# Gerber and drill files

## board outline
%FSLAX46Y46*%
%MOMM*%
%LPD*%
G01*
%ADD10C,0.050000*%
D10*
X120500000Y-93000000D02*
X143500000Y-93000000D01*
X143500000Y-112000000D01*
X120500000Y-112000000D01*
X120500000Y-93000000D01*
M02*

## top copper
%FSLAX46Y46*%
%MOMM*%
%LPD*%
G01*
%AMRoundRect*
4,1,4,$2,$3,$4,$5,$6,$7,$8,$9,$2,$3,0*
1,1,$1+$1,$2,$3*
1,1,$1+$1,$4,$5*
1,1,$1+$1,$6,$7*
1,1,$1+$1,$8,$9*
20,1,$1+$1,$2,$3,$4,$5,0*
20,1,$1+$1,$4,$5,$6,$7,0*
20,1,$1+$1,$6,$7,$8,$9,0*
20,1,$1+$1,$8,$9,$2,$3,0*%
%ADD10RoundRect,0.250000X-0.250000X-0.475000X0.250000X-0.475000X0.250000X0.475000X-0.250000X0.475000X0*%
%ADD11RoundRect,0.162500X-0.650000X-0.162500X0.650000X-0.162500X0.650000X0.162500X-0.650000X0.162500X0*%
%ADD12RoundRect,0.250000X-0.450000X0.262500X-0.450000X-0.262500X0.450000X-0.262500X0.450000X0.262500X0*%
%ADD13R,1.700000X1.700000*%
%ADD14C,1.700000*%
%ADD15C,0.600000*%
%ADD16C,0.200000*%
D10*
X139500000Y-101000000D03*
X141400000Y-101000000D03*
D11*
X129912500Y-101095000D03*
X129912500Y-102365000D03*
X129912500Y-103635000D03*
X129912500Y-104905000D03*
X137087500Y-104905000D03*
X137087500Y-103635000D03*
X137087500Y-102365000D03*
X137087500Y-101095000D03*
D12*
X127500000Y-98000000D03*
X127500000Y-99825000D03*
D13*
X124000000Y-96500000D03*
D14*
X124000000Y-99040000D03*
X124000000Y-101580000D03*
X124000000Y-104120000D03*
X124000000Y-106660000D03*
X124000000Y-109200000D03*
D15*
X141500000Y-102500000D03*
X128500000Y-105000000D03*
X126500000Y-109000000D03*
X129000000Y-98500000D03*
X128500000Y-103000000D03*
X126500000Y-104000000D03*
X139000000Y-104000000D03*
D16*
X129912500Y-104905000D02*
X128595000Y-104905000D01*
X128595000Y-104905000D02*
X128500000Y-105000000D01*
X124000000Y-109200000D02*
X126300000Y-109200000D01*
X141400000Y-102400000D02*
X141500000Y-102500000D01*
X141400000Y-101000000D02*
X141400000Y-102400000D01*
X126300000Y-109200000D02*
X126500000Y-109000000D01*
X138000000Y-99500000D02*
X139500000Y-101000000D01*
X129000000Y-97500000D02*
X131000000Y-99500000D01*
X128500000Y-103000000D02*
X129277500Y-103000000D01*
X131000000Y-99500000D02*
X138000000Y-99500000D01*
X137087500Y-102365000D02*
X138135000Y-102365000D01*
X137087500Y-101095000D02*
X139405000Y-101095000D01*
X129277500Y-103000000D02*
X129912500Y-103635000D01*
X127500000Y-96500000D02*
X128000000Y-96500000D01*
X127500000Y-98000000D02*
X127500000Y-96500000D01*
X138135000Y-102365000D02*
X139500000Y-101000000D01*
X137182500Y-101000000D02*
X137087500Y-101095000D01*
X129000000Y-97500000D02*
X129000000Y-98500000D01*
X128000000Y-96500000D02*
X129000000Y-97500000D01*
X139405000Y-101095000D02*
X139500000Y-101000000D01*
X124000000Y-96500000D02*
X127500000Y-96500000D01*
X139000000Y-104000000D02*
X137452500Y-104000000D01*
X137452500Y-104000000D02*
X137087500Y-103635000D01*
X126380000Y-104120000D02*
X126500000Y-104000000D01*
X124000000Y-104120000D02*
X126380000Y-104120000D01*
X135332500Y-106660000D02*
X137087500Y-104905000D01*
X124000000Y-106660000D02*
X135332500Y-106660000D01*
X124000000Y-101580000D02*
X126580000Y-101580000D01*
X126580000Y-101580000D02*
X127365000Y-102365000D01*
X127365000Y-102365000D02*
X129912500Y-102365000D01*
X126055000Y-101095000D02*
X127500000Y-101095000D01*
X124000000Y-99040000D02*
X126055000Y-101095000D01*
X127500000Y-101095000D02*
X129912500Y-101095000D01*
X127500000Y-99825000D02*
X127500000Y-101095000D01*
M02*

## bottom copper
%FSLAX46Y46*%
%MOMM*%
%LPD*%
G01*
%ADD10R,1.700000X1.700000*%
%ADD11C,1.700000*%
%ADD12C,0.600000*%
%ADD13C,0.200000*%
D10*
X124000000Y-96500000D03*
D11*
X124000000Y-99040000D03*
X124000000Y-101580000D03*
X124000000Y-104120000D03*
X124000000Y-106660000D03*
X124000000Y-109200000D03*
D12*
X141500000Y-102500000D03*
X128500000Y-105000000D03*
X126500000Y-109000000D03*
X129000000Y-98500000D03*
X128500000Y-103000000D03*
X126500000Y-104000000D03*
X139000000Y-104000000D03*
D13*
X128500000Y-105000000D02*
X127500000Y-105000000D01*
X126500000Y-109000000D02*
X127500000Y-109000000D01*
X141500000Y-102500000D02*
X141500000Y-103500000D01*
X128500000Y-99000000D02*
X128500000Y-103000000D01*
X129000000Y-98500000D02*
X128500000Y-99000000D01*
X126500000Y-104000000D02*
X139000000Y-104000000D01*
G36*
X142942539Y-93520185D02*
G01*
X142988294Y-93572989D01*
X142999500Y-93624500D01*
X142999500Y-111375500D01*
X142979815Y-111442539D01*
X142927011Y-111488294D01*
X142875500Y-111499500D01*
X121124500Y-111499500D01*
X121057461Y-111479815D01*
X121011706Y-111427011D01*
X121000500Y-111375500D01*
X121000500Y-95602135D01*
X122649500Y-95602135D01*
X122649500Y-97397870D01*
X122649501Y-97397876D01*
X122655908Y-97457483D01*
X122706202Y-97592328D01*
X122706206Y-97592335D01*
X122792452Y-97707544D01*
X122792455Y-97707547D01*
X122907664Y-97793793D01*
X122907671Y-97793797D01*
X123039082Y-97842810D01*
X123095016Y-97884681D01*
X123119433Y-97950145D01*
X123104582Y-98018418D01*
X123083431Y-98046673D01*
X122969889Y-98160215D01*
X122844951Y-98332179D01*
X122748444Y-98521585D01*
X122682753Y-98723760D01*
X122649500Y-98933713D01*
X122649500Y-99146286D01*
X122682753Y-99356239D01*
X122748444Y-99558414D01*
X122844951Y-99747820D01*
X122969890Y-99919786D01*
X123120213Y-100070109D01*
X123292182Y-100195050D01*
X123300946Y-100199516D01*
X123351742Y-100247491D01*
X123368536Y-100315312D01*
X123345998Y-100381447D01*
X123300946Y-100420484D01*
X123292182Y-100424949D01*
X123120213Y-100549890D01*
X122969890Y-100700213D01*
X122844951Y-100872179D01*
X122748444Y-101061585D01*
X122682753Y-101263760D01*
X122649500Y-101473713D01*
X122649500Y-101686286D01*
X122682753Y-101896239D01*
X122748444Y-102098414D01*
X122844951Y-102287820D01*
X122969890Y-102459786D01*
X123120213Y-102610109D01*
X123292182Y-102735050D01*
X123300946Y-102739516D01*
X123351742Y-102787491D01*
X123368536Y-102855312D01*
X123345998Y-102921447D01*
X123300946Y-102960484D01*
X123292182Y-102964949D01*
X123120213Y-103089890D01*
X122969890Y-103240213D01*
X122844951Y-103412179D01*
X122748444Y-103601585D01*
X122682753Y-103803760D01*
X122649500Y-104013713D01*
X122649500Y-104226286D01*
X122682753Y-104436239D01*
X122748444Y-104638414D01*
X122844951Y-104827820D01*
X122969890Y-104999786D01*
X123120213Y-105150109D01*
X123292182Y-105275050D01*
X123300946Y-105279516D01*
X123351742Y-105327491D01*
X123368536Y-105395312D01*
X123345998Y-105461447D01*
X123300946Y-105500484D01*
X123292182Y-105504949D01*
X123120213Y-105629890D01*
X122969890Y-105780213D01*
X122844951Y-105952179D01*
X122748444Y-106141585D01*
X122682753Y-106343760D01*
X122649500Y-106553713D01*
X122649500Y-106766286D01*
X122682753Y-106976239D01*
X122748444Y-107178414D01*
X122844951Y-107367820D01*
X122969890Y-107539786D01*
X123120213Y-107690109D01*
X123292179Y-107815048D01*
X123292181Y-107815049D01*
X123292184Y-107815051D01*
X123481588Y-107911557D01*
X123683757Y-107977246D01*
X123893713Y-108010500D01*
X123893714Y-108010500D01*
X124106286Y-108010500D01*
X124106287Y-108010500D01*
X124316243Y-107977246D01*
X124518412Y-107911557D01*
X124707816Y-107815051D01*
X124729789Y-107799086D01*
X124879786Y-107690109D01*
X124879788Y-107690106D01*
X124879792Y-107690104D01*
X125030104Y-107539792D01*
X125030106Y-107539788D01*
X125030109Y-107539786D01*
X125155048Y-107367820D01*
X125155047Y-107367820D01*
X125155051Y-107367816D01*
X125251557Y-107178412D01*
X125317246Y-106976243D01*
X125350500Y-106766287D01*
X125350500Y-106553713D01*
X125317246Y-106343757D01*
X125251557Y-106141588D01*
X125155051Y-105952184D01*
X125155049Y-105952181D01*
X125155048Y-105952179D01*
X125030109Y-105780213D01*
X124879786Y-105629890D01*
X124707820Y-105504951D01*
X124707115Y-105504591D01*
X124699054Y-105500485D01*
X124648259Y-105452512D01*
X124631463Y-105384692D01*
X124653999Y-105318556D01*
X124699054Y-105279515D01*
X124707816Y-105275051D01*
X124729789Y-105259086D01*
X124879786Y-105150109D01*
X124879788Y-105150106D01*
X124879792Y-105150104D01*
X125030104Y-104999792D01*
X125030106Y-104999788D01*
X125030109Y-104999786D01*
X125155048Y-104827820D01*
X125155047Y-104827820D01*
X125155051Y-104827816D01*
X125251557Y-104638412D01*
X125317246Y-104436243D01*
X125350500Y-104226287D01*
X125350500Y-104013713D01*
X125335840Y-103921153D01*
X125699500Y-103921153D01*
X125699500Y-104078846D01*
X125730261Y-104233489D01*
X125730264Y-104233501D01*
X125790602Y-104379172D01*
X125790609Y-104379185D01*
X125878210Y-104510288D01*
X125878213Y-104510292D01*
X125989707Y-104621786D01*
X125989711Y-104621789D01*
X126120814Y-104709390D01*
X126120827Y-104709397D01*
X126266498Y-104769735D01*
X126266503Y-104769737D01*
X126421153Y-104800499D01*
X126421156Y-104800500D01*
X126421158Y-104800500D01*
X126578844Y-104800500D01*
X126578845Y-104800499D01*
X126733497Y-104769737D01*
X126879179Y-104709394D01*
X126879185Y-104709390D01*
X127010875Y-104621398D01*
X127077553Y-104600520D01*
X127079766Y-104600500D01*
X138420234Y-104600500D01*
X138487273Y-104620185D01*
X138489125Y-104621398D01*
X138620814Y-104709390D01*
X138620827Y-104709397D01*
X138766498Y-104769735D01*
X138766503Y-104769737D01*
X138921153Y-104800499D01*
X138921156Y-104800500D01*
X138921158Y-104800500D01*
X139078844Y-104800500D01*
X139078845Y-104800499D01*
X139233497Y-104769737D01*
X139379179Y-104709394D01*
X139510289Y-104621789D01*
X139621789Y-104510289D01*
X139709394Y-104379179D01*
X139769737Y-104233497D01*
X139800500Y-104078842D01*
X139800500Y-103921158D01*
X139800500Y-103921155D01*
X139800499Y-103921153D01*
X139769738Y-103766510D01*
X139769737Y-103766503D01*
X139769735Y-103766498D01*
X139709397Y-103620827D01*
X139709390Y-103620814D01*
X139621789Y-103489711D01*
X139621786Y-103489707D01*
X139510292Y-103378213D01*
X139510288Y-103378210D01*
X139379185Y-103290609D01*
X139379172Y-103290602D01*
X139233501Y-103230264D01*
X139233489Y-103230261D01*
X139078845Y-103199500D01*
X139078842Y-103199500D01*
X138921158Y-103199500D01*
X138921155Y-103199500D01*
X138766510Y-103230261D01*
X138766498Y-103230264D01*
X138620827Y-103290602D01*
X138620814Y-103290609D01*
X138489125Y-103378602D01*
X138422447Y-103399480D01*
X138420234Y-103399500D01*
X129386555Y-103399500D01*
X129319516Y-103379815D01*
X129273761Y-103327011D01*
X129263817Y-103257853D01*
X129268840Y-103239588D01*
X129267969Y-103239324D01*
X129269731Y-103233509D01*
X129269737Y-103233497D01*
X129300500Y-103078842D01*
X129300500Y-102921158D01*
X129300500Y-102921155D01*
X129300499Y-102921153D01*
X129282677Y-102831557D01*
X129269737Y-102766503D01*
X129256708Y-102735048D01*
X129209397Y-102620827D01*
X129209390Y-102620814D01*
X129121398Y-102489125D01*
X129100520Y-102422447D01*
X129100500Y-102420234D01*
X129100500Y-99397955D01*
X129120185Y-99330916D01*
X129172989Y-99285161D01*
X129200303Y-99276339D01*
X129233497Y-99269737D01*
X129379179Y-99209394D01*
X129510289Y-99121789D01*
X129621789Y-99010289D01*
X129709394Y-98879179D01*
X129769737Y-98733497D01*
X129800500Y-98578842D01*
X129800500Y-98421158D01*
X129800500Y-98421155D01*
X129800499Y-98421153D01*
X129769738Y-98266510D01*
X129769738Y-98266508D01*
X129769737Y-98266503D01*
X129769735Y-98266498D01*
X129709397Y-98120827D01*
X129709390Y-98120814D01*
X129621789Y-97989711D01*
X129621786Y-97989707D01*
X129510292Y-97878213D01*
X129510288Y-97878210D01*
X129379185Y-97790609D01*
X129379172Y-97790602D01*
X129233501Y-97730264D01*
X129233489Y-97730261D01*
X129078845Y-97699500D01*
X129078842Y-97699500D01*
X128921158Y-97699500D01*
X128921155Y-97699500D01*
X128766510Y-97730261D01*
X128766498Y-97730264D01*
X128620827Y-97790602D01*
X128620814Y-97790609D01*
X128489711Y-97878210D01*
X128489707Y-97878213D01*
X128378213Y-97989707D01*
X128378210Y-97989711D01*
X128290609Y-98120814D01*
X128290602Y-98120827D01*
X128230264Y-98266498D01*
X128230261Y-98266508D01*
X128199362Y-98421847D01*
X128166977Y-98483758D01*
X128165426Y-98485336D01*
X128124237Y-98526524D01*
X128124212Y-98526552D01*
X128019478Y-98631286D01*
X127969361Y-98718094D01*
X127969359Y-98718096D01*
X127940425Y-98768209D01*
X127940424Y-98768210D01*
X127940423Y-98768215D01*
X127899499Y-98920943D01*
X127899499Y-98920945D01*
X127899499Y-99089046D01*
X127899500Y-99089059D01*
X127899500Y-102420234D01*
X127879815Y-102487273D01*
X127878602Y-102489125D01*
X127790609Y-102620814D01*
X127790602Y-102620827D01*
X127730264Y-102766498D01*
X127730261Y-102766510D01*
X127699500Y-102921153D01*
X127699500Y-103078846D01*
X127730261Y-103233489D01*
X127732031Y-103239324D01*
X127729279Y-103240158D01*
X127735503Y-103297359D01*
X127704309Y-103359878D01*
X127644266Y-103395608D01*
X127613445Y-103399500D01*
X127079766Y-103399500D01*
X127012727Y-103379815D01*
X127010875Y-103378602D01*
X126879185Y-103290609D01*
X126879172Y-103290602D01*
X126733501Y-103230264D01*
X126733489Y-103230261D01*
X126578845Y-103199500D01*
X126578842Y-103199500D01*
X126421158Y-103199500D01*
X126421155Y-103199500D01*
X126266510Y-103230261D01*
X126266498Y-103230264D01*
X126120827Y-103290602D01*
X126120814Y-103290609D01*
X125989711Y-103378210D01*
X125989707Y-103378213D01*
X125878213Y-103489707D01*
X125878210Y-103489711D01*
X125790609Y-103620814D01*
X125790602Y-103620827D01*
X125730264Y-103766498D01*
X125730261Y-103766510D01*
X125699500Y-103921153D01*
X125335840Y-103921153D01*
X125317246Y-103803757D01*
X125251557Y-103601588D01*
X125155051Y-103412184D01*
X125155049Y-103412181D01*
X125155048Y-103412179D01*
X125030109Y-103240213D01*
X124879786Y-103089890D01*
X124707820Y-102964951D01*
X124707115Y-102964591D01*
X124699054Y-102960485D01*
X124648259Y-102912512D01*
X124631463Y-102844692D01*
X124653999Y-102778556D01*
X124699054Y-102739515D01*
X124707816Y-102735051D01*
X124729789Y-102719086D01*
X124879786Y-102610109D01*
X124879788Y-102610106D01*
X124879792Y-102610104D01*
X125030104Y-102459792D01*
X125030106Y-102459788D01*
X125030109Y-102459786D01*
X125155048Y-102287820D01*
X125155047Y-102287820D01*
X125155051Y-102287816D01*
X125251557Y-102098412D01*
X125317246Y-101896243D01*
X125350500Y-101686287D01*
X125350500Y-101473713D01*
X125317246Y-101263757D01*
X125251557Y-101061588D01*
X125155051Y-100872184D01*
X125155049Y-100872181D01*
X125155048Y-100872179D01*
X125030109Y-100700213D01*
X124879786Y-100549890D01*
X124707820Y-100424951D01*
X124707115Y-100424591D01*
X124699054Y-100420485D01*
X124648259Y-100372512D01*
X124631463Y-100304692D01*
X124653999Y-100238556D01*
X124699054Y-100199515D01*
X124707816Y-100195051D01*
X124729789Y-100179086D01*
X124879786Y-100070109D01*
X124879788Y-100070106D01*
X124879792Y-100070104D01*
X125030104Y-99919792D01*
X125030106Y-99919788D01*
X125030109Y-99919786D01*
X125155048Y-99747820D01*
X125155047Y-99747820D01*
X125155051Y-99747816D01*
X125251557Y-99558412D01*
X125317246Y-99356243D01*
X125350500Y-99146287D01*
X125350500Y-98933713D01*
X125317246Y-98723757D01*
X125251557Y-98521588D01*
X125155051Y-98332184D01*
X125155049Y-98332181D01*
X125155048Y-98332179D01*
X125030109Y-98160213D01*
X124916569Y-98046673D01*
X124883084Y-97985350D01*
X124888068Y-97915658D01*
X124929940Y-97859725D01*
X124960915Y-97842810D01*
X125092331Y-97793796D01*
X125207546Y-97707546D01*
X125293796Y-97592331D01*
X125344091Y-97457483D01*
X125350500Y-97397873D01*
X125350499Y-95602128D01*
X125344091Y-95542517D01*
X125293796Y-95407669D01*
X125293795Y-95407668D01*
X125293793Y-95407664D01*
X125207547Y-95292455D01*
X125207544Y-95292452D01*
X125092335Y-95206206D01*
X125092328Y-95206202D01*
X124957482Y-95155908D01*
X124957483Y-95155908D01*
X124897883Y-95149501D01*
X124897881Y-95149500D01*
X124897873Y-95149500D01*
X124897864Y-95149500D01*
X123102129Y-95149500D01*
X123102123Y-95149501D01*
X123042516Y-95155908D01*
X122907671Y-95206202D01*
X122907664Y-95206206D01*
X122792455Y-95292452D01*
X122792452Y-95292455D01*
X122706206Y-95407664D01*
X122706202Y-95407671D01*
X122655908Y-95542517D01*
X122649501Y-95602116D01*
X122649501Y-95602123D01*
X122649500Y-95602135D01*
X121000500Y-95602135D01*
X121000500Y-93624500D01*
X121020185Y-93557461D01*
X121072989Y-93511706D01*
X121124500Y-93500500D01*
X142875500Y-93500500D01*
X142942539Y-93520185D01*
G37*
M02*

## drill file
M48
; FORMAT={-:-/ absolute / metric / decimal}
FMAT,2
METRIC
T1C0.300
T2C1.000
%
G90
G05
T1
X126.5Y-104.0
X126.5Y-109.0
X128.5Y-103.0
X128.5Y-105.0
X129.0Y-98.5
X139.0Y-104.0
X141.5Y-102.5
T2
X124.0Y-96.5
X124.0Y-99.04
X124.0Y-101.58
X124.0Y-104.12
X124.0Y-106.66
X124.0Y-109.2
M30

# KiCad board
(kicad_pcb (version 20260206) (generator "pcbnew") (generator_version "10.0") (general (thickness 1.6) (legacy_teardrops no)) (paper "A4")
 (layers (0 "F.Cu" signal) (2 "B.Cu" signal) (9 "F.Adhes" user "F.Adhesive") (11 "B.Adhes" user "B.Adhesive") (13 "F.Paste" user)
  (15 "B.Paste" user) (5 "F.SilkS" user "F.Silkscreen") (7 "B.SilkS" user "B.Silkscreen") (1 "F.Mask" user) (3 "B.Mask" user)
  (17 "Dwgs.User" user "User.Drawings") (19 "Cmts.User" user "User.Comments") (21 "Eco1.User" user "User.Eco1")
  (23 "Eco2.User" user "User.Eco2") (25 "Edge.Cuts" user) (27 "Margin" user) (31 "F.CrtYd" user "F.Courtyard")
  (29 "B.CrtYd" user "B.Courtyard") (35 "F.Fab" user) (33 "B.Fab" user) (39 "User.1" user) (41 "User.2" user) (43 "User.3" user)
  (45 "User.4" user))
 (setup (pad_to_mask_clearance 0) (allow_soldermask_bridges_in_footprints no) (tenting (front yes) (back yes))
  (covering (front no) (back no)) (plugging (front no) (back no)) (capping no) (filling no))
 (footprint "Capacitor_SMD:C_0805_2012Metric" (layer "F.Cu") (at 140.45 101)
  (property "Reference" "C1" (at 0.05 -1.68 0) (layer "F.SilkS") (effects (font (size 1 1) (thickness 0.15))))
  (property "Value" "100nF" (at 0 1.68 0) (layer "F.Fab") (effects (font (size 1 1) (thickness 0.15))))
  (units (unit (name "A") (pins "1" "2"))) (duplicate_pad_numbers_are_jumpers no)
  (pad "1" smd roundrect (at -0.95 0) (size 1 1.45) (layers "F.Cu" "F.Mask" "F.Paste") (roundrect_rratio 0.25) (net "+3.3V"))
  (pad "2" smd roundrect (at 0.95 0) (size 1 1.45) (layers "F.Cu" "F.Mask" "F.Paste") (roundrect_rratio 0.25) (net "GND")))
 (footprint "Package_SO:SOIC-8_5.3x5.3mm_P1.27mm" (layer "F.Cu") (at 133.5 103)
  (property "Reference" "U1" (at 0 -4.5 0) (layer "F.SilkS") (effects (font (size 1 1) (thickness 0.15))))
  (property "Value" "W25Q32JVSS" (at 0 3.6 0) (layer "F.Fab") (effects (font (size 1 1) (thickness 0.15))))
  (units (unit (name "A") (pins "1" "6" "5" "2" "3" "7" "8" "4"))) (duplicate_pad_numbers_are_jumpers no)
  (pad "1" smd roundrect (at -3.5875 -1.905) (size 1.625 0.65) (layers "F.Cu" "F.Mask" "F.Paste") (roundrect_rratio 0.25)
   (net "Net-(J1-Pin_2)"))
  (pad "2" smd roundrect (at -3.5875 -0.635) (size 1.625 0.65) (layers "F.Cu" "F.Mask" "F.Paste") (roundrect_rratio 0.25)
   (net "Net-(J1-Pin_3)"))
  (pad "3" smd roundrect (at -3.5875 0.635) (size 1.625 0.65) (layers "F.Cu" "F.Mask" "F.Paste") (roundrect_rratio 0.25) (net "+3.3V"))
  (pad "4" smd roundrect (at -3.5875 1.905) (size 1.625 0.65) (layers "F.Cu" "F.Mask" "F.Paste") (roundrect_rratio 0.25) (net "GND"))
  (pad "5" smd roundrect (at 3.5875 1.905) (size 1.625 0.65) (layers "F.Cu" "F.Mask" "F.Paste") (roundrect_rratio 0.25)
   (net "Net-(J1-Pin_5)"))
  (pad "6" smd roundrect (at 3.5875 0.635) (size 1.625 0.65) (layers "F.Cu" "F.Mask" "F.Paste") (roundrect_rratio 0.25)
   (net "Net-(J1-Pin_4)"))
  (pad "7" smd roundrect (at 3.5875 -0.635) (size 1.625 0.65) (layers "F.Cu" "F.Mask" "F.Paste") (roundrect_rratio 0.25) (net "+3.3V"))
  (pad "8" smd roundrect (at 3.5875 -1.905) (size 1.625 0.65) (layers "F.Cu" "F.Mask" "F.Paste") (roundrect_rratio 0.25) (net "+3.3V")))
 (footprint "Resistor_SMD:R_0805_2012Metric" (layer "F.Cu") (at 127.5 98.9125 -90)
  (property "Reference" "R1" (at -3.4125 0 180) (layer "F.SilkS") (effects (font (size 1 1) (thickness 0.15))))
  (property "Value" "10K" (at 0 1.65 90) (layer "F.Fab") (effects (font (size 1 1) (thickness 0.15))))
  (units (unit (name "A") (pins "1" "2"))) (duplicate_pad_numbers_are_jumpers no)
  (pad "1" smd roundrect (at -0.9125 0 270) (size 1.025 1.4) (layers "F.Cu" "F.Mask" "F.Paste") (roundrect_rratio 0.243902) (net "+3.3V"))
  (pad "2" smd roundrect (at 0.9125 0 270) (size 1.025 1.4) (layers "F.Cu" "F.Mask" "F.Paste") (roundrect_rratio 0.243902)
   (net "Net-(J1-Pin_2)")))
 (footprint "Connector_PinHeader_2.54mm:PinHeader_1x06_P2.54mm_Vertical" (layer "F.Cu") (at 124 96.5)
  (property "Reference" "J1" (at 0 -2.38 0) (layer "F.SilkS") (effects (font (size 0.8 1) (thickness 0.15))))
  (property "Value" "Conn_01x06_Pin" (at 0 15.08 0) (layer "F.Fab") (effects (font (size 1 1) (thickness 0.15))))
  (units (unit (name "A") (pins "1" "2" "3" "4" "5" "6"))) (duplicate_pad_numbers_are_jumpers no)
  (pad "1" thru_hole rect (at 0 0) (size 1.7 1.7) (drill 1) (layers "*.Cu" "*.Mask") (remove_unused_layers no) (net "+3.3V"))
  (pad "2" thru_hole circle (at 0 2.54) (size 1.7 1.7) (drill 1) (layers "*.Cu" "*.Mask") (remove_unused_layers no) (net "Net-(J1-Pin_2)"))
  (pad "3" thru_hole circle (at 0 5.08) (size 1.7 1.7) (drill 1) (layers "*.Cu" "*.Mask") (remove_unused_layers no) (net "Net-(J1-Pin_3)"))
  (pad "4" thru_hole circle (at 0 7.62) (size 1.7 1.7) (drill 1) (layers "*.Cu" "*.Mask") (remove_unused_layers no) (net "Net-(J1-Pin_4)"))
  (pad "5" thru_hole circle (at 0 10.16) (size 1.7 1.7) (drill 1) (layers "*.Cu" "*.Mask") (remove_unused_layers no) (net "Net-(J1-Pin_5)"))
  (pad "6" thru_hole circle (at 0 12.7) (size 1.7 1.7) (drill 1) (layers "*.Cu" "*.Mask") (remove_unused_layers no) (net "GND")))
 (gr_rect (start 120.5 93) (end 143.5 112) (stroke (width 0.05) (type default)) (fill no) (layer "Edge.Cuts"))
 (segment (start 129.9125 104.905) (end 128.595 104.905) (width 0.2) (layer "F.Cu") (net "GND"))
 (segment (start 128.595 104.905) (end 128.5 105) (width 0.2) (layer "F.Cu") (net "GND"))
 (segment (start 124 109.2) (end 126.3 109.2) (width 0.2) (layer "F.Cu") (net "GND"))
 (segment (start 141.4 102.4) (end 141.5 102.5) (width 0.2) (layer "F.Cu") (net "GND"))
 (segment (start 141.4 101) (end 141.4 102.4) (width 0.2) (layer "F.Cu") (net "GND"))
 (segment (start 126.3 109.2) (end 126.5 109) (width 0.2) (layer "F.Cu") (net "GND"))
 (via (at 141.5 102.5) (size 0.6) (drill 0.3) (layers "F.Cu" "B.Cu") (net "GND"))
 (via (at 128.5 105) (size 0.6) (drill 0.3) (layers "F.Cu" "B.Cu") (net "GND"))
 (via (at 126.5 109) (size 0.6) (drill 0.3) (layers "F.Cu" "B.Cu") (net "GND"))
 (segment (start 128.5 105) (end 127.5 105) (width 0.2) (layer "B.Cu") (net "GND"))
 (segment (start 126.5 109) (end 127.5 109) (width 0.2) (layer "B.Cu") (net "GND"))
 (segment (start 141.5 102.5) (end 141.5 103.5) (width 0.2) (layer "B.Cu") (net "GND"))
 (segment (start 138 99.5) (end 139.5 101) (width 0.2) (layer "F.Cu") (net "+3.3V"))
 (segment (start 129 97.5) (end 131 99.5) (width 0.2) (layer "F.Cu") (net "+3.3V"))
 (segment (start 128.5 103) (end 129.2775 103) (width 0.2) (layer "F.Cu") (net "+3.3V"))
 (segment (start 131 99.5) (end 138 99.5) (width 0.2) (layer "F.Cu") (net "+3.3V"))
 (segment (start 137.0875 102.365) (end 138.135 102.365) (width 0.2) (layer "F.Cu") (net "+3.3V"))
 (segment (start 137.0875 101.095) (end 139.405 101.095) (width 0.2) (layer "F.Cu") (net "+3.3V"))
 (segment (start 129.2775 103) (end 129.9125 103.635) (width 0.2) (layer "F.Cu") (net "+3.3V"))
 (segment (start 127.5 96.5) (end 128 96.5) (width 0.2) (layer "F.Cu") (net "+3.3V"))
 (segment (start 127.5 98) (end 127.5 96.5) (width 0.2) (layer "F.Cu") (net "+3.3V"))
 (segment (start 138.135 102.365) (end 139.5 101) (width 0.2) (layer "F.Cu") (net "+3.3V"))
 (segment (start 137.1825 101) (end 137.0875 101.095) (width 0.2) (layer "F.Cu") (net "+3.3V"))
 (segment (start 129 97.5) (end 129 98.5) (width 0.2) (layer "F.Cu") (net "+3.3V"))
 (segment (start 128 96.5) (end 129 97.5) (width 0.2) (layer "F.Cu") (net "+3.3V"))
 (segment (start 139.405 101.095) (end 139.5 101) (width 0.2) (layer "F.Cu") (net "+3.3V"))
 (segment (start 124 96.5) (end 127.5 96.5) (width 0.2) (layer "F.Cu") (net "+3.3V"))
 (via (at 129 98.5) (size 0.6) (drill 0.3) (layers "F.Cu" "B.Cu") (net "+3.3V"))
 (via (at 128.5 103) (size 0.6) (drill 0.3) (layers "F.Cu" "B.Cu") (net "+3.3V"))
 (segment (start 128.5 99) (end 128.5 103) (width 0.2) (layer "B.Cu") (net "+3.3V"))
 (segment (start 129 98.5) (end 128.5 99) (width 0.2) (layer "B.Cu") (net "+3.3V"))
 (segment (start 139 104) (end 137.4525 104) (width 0.2) (layer "F.Cu") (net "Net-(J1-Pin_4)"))
 (segment (start 137.4525 104) (end 137.0875 103.635) (width 0.2) (layer "F.Cu") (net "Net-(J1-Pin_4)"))
 (segment (start 126.38 104.12) (end 126.5 104) (width 0.2) (layer "F.Cu") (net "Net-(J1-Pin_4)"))
 (segment (start 124 104.12) (end 126.38 104.12) (width 0.2) (layer "F.Cu") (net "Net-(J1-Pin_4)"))
 (via (at 126.5 104) (size 0.6) (drill 0.3) (layers "F.Cu" "B.Cu") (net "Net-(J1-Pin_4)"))
 (via (at 139 104) (size 0.6) (drill 0.3) (layers "F.Cu" "B.Cu") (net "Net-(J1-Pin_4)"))
 (segment (start 126.5 104) (end 139 104) (width 0.2) (layer "B.Cu") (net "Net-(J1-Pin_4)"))
 (segment (start 135.3325 106.66) (end 137.0875 104.905) (width 0.2) (layer "F.Cu") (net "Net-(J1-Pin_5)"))
 (segment (start 124 106.66) (end 135.3325 106.66) (width 0.2) (layer "F.Cu") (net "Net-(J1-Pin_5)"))
 (segment (start 124 101.58) (end 126.58 101.58) (width 0.2) (layer "F.Cu") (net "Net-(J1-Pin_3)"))
 (segment (start 126.58 101.58) (end 127.365 102.365) (width 0.2) (layer "F.Cu") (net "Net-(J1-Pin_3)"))
 (segment (start 127.365 102.365) (end 129.9125 102.365) (width 0.2) (layer "F.Cu") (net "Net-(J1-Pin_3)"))
 (segment (start 126.055 101.095) (end 127.5 101.095) (width 0.2) (layer "F.Cu") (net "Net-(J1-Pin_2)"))
 (segment (start 124 99.04) (end 126.055 101.095) (width 0.2) (layer "F.Cu") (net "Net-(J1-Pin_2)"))
 (segment (start 127.5 101.095) (end 129.9125 101.095) (width 0.2) (layer "F.Cu") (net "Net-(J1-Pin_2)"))
 (segment (start 127.5 99.825) (end 127.5 101.095) (width 0.2) (layer "F.Cu") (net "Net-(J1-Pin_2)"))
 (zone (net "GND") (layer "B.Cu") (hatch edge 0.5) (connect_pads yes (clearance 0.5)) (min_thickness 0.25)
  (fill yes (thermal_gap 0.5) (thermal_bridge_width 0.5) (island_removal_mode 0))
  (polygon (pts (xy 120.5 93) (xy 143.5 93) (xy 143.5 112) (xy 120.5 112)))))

